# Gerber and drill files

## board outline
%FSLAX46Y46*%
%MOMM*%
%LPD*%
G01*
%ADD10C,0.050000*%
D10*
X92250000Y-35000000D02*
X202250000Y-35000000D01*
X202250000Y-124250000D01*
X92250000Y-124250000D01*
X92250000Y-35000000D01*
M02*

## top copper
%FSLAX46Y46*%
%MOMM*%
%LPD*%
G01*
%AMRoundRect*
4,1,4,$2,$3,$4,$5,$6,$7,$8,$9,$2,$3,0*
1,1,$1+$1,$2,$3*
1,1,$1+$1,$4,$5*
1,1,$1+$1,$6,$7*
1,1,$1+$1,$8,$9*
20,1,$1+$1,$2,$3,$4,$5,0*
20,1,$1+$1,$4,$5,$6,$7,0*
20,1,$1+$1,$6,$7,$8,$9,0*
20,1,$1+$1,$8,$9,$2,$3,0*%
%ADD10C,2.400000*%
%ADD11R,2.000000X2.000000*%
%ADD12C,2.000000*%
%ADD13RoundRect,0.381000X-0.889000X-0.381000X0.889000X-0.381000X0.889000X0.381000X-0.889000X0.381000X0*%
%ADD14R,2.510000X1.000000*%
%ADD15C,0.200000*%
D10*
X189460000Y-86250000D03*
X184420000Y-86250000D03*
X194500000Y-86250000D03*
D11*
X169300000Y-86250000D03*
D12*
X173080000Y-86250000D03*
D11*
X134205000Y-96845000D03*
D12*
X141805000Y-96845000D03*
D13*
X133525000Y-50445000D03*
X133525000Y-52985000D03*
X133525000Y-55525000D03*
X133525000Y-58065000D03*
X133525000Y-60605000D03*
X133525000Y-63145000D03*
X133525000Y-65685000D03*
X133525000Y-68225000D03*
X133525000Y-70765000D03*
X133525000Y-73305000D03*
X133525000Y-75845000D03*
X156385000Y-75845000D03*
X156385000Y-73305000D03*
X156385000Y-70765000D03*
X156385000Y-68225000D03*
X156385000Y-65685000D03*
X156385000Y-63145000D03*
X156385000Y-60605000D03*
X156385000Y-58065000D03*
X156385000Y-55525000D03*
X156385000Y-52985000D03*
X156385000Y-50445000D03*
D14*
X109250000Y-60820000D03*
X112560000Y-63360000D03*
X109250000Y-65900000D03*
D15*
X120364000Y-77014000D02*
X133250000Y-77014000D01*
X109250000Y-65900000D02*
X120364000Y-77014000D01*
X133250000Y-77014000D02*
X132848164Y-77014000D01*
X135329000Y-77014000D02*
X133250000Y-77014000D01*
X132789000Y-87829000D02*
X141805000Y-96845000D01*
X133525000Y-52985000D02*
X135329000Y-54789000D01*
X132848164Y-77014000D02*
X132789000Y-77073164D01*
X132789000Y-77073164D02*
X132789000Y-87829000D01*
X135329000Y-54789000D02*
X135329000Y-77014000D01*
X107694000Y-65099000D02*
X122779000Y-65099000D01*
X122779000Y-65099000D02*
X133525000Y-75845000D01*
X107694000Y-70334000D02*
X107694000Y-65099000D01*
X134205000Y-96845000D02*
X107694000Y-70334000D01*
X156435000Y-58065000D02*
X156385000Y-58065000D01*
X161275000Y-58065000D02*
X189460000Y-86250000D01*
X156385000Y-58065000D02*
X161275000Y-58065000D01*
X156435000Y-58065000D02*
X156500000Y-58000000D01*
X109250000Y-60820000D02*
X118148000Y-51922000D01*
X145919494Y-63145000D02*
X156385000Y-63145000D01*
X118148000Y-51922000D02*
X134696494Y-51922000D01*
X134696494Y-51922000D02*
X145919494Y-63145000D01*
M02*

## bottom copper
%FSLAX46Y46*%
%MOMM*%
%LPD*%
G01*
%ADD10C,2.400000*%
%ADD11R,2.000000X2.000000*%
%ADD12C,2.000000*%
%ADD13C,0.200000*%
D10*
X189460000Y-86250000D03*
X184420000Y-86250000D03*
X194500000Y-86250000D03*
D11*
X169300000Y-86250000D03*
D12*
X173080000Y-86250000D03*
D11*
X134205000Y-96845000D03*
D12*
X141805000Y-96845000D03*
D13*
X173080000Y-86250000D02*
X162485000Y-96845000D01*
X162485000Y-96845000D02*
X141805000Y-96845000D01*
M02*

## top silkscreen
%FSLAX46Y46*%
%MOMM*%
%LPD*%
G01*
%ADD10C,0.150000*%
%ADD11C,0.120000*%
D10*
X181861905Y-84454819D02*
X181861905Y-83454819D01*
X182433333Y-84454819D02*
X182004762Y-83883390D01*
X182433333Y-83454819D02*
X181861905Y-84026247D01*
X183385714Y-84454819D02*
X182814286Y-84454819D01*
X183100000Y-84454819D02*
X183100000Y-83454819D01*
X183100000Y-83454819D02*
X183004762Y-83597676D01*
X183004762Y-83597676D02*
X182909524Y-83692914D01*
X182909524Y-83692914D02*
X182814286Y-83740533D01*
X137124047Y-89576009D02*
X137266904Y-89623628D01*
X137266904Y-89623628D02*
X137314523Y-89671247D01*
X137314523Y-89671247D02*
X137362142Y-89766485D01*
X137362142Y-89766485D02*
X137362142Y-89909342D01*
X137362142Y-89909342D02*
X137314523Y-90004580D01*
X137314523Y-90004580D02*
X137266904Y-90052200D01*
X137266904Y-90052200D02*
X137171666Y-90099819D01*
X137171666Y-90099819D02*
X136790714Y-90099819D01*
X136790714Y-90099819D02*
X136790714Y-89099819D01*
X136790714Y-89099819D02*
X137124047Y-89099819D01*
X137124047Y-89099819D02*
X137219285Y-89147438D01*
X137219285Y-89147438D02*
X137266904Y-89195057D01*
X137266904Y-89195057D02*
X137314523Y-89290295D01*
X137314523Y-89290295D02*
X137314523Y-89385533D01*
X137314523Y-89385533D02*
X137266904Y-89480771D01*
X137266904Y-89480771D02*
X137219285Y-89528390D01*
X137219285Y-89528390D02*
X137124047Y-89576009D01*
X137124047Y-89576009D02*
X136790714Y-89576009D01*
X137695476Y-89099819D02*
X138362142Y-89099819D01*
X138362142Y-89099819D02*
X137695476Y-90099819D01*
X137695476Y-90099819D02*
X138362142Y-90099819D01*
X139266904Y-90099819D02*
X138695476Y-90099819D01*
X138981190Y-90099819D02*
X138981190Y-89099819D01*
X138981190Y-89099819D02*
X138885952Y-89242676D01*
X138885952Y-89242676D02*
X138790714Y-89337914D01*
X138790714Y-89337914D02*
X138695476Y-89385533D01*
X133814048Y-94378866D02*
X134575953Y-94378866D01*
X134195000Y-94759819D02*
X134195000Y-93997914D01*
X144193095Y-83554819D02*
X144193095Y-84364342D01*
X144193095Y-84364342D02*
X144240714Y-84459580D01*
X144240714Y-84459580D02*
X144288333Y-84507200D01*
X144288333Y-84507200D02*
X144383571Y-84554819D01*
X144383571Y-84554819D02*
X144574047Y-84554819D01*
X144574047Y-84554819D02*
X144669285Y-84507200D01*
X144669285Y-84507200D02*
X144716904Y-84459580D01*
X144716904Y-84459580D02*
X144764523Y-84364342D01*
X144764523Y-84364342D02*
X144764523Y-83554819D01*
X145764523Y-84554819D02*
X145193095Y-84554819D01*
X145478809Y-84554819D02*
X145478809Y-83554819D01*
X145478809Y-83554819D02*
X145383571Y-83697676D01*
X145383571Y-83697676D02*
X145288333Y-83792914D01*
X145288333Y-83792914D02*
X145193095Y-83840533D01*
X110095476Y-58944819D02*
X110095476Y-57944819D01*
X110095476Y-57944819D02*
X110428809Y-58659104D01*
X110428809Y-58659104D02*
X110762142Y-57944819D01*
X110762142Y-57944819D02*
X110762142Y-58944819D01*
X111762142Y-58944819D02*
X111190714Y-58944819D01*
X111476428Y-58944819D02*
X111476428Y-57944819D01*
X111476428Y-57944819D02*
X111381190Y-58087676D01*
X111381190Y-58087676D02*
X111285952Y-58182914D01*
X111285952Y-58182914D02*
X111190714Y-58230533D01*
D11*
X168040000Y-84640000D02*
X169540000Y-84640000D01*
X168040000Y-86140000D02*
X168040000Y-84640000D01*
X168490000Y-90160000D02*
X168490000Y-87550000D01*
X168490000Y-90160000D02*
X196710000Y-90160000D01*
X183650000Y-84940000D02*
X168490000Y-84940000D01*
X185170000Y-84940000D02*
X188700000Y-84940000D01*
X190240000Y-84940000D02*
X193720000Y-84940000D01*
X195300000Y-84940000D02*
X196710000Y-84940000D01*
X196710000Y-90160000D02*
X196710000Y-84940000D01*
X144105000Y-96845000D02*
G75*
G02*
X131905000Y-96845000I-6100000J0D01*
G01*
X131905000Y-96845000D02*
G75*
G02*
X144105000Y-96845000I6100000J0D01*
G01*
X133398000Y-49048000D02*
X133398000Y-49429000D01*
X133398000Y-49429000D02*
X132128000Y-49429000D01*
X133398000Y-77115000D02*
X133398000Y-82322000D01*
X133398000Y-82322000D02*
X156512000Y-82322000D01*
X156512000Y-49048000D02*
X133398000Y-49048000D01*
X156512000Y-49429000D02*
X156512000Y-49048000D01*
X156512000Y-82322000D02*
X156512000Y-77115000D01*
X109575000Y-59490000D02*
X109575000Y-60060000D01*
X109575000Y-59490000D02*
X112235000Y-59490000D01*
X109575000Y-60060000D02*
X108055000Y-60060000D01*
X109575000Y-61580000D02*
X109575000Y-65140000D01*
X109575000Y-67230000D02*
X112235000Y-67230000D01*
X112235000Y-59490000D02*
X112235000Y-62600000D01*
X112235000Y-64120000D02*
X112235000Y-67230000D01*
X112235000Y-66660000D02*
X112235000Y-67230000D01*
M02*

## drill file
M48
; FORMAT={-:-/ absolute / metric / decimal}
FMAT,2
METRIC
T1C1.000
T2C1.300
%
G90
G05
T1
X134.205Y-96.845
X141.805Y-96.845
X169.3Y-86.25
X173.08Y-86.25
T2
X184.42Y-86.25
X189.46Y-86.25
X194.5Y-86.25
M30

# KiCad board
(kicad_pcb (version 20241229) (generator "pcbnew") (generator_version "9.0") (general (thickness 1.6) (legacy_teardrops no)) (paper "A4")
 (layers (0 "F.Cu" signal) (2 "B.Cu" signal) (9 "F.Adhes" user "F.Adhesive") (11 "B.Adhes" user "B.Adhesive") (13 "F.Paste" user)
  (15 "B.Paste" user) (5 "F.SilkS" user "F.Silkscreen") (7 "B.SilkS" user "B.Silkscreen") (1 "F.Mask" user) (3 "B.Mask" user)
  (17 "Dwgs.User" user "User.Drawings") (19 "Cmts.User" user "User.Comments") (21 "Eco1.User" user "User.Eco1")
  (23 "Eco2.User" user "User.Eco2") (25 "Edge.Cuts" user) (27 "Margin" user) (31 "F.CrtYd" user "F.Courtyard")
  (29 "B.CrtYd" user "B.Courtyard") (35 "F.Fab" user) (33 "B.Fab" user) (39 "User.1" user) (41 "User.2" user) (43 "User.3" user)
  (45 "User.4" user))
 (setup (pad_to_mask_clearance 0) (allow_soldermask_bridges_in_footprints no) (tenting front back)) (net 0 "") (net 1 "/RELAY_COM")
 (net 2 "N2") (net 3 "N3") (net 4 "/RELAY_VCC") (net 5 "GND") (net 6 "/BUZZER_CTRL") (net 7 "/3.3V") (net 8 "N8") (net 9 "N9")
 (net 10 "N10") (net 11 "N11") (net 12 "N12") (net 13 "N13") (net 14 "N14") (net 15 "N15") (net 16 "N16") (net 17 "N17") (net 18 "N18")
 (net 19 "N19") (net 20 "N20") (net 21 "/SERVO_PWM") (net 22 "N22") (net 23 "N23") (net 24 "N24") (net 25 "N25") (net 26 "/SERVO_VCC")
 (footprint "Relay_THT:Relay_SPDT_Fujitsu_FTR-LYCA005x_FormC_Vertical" (layer "F.Cu") (at 169.3 86.25)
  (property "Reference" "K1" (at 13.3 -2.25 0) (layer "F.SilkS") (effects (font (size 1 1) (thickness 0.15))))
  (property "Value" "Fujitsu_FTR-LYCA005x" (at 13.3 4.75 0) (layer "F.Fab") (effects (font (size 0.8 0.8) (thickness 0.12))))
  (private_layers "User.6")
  (fp_line (start -1.26 -1.61) (end 0.24 -1.61) (stroke (width 0.12) (type solid)) (layer "F.SilkS"))
  (fp_line (start -1.26 -0.11) (end -1.26 -1.61) (stroke (width 0.12) (type solid)) (layer "F.SilkS"))
  (fp_line (start -0.81 3.91) (end -0.81 1.3) (stroke (width 0.12) (type solid)) (layer "F.SilkS"))
  (fp_line (start -0.81 3.91) (end 27.41 3.91) (stroke (width 0.12) (type solid)) (layer "F.SilkS"))
  (fp_line (start 14.35 -1.31) (end -0.81 -1.31) (stroke (width 0.12) (type solid)) (layer "F.SilkS"))
  (fp_line (start 15.87 -1.31) (end 19.4 -1.31) (stroke (width 0.12) (type solid)) (layer "F.SilkS"))
  (fp_line (start 20.94 -1.31) (end 24.42 -1.31) (stroke (width 0.12) (type solid)) (layer "F.SilkS"))
  (fp_line (start 26 -1.31) (end 27.41 -1.31) (stroke (width 0.12) (type solid)) (layer "F.SilkS"))
  (fp_line (start 27.41 3.91) (end 27.41 -1.31) (stroke (width 0.12) (type solid)) (layer "F.SilkS"))
  (pad "11" thru_hole circle (at 20.16 0) (size 2.4 2.4) (drill 1.3) (layers "*.Cu" "*.Mask") (remove_unused_layers no) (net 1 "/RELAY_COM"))
  (pad "12" thru_hole circle (at 15.12 0) (size 2.4 2.4) (drill 1.3) (layers "*.Cu" "*.Mask") (remove_unused_layers no) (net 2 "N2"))
  (pad "14" thru_hole circle (at 25.2 0) (size 2.4 2.4) (drill 1.3) (layers "*.Cu" "*.Mask") (remove_unused_layers no) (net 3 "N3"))
  (pad "A1" thru_hole rect (at 0 0) (size 2 2) (drill 1) (layers "*.Cu" "*.Mask") (remove_unused_layers no) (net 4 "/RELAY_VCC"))
  (pad "A2" thru_hole circle (at 3.78 0) (size 2 2) (drill 1) (layers "*.Cu" "*.Mask") (remove_unused_layers no) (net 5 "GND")))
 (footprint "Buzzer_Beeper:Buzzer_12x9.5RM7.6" (layer "F.Cu") (at 134.205 96.845)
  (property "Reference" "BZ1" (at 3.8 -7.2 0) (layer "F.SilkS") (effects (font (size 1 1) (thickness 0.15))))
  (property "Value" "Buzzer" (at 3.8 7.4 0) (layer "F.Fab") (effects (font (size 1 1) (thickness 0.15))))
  (fp_circle (center 3.8 0) (end 9.9 0) (stroke (width 0.12) (type solid)) (fill no) (layer "F.SilkS"))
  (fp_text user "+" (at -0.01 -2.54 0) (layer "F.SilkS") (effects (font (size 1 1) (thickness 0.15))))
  (pad "1" thru_hole rect (at 0 0) (size 2 2) (drill 1) (layers "*.Cu" "*.Mask") (remove_unused_layers no) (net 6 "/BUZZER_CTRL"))
  (pad "2" thru_hole circle (at 7.6 0) (size 2 2) (drill 1) (layers "*.Cu" "*.Mask") (remove_unused_layers no) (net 5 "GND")))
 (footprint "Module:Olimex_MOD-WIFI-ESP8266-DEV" (layer "F.Cu") (at 144.955 63.145)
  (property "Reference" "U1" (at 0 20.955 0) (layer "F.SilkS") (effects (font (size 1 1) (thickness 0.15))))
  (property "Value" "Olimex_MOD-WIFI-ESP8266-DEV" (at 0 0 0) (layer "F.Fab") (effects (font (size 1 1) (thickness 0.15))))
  (fp_line (start -11.557 -14.097) (end -11.557 -13.716) (stroke (width 0.12) (type solid)) (layer "F.SilkS"))
  (fp_line (start -11.557 -13.716) (end -12.827 -13.716) (stroke (width 0.12) (type solid)) (layer "F.SilkS"))
  (fp_line (start -11.557 13.97) (end -11.557 19.177) (stroke (width 0.12) (type solid)) (layer "F.SilkS"))
  (fp_line (start -11.557 19.177) (end 11.557 19.177) (stroke (width 0.12) (type solid)) (layer "F.SilkS"))
  (fp_line (start 11.557 -14.097) (end -11.557 -14.097) (stroke (width 0.12) (type solid)) (layer "F.SilkS"))
  (fp_line (start 11.557 -13.716) (end 11.557 -14.097) (stroke (width 0.12) (type solid)) (layer "F.SilkS"))
  (fp_line (start 11.557 19.177) (end 11.557 13.97) (stroke (width 0.12) (type solid)) (layer "F.SilkS"))
  (pad "1" smd roundrect (at -11.43 -12.7) (size 2.54 1.524) (layers "F.Cu" "F.Mask" "F.Paste") (roundrect_rratio 0.25) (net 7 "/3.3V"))
  (pad "2" smd roundrect (at -11.43 -10.16) (size 2.54 1.524) (layers "F.Cu" "F.Mask" "F.Paste") (roundrect_rratio 0.25) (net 5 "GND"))
  (pad "3" smd roundrect (at -11.43 -7.62) (size 2.54 1.524) (layers "F.Cu" "F.Mask" "F.Paste") (roundrect_rratio 0.25) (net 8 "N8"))
  (pad "4" smd roundrect (at -11.43 -5.08) (size 2.54 1.524) (layers "F.Cu" "F.Mask" "F.Paste") (roundrect_rratio 0.25) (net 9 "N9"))
  (pad "5" smd roundrect (at -11.43 -2.54) (size 2.54 1.524) (layers "F.Cu" "F.Mask" "F.Paste") (roundrect_rratio 0.25) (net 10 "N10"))
  (pad "6" smd roundrect (at -11.43 0) (size 2.54 1.524) (layers "F.Cu" "F.Mask" "F.Paste") (roundrect_rratio 0.25) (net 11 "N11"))
  (pad "7" smd roundrect (at -11.43 2.54) (size 2.54 1.524) (layers "F.Cu" "F.Mask" "F.Paste") (roundrect_rratio 0.25) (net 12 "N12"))
  (pad "8" smd roundrect (at -11.43 5.08) (size 2.54 1.524) (layers "F.Cu" "F.Mask" "F.Paste") (roundrect_rratio 0.25) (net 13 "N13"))
  (pad "9" smd roundrect (at -11.43 7.62) (size 2.54 1.524) (layers "F.Cu" "F.Mask" "F.Paste") (roundrect_rratio 0.25) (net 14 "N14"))
  (pad "10" smd roundrect (at -11.43 10.16) (size 2.54 1.524) (layers "F.Cu" "F.Mask" "F.Paste") (roundrect_rratio 0.25) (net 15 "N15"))
  (pad "11" smd roundrect (at -11.43 12.7) (size 2.54 1.524) (layers "F.Cu" "F.Mask" "F.Paste") (roundrect_rratio 0.25)
   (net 6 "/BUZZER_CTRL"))
  (pad "12" smd roundrect (at 11.43 12.7) (size 2.54 1.524) (layers "F.Cu" "F.Mask" "F.Paste") (roundrect_rratio 0.25) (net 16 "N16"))
  (pad "13" smd roundrect (at 11.43 10.16) (size 2.54 1.524) (layers "F.Cu" "F.Mask" "F.Paste") (roundrect_rratio 0.25) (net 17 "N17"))
  (pad "14" smd roundrect (at 11.43 7.62) (size 2.54 1.524) (layers "F.Cu" "F.Mask" "F.Paste") (roundrect_rratio 0.25) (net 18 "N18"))
  (pad "15" smd roundrect (at 11.43 5.08) (size 2.54 1.524) (layers "F.Cu" "F.Mask" "F.Paste") (roundrect_rratio 0.25) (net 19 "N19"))
  (pad "16" smd roundrect (at 11.43 2.54) (size 2.54 1.524) (layers "F.Cu" "F.Mask" "F.Paste") (roundrect_rratio 0.25) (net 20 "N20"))
  (pad "17" smd roundrect (at 11.43 0) (size 2.54 1.524) (layers "F.Cu" "F.Mask" "F.Paste") (roundrect_rratio 0.25) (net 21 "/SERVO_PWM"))
  (pad "18" smd roundrect (at 11.43 -2.54) (size 2.54 1.524) (layers "F.Cu" "F.Mask" "F.Paste") (roundrect_rratio 0.25) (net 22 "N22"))
  (pad "19" smd roundrect (at 11.43 -5.08) (size 2.54 1.524) (layers "F.Cu" "F.Mask" "F.Paste") (roundrect_rratio 0.25) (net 1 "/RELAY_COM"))
  (pad "20" smd roundrect (at 11.43 -7.62) (size 2.54 1.524) (layers "F.Cu" "F.Mask" "F.Paste") (roundrect_rratio 0.25) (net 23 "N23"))
  (pad "21" smd roundrect (at 11.43 -10.16) (size 2.54 1.524) (layers "F.Cu" "F.Mask" "F.Paste") (roundrect_rratio 0.25) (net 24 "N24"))
  (pad "22" smd roundrect (at 11.43 -12.7) (size 2.54 1.524) (layers "F.Cu" "F.Mask" "F.Paste") (roundrect_rratio 0.25) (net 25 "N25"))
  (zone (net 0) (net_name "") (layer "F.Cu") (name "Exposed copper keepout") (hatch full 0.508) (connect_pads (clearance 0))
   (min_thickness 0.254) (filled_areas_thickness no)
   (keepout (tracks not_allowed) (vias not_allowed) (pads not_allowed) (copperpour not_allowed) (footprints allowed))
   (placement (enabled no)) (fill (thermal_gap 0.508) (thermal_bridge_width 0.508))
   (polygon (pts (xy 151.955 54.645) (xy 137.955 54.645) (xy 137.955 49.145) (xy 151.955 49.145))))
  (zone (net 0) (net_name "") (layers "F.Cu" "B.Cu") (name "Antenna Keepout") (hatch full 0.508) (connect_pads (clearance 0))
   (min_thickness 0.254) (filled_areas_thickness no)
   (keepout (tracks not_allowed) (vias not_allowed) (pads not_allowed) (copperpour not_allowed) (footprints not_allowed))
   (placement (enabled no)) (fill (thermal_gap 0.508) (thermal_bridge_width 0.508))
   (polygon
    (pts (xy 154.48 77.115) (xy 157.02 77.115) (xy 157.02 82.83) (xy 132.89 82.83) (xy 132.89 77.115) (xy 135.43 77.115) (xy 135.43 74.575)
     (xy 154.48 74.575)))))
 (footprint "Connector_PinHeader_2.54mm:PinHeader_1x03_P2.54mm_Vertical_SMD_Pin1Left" (layer "F.Cu") (at 110.905 63.36)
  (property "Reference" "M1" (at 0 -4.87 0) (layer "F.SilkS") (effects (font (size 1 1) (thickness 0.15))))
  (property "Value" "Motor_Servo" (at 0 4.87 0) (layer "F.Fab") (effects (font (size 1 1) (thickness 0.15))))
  (fp_line (start -1.33 -3.87) (end -1.33 -3.3) (stroke (width 0.12) (type solid)) (layer "F.SilkS"))
  (fp_line (start -1.33 -3.87) (end 1.33 -3.87) (stroke (width 0.12) (type solid)) (layer "F.SilkS"))
  (fp_line (start -1.33 -3.3) (end -2.85 -3.3) (stroke (width 0.12) (type solid)) (layer "F.SilkS"))
  (fp_line (start -1.33 -1.78) (end -1.33 1.78) (stroke (width 0.12) (type solid)) (layer "F.SilkS"))
  (fp_line (start -1.33 3.87) (end 1.33 3.87) (stroke (width 0.12) (type solid)) (layer "F.SilkS"))
  (fp_line (start 1.33 -3.87) (end 1.33 -0.76) (stroke (width 0.12) (type solid)) (layer "F.SilkS"))
  (fp_line (start 1.33 0.76) (end 1.33 3.87) (stroke (width 0.12) (type solid)) (layer "F.SilkS"))
  (fp_line (start 1.33 3.3) (end 1.33 3.87) (stroke (width 0.12) (type solid)) (layer "F.SilkS"))
  (pad "1" smd rect (at -1.655 -2.54) (size 2.51 1) (layers "F.Cu" "F.Mask" "F.Paste") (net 21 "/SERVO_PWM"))
  (pad "2" smd rect (at 1.655 0) (size 2.51 1) (layers "F.Cu" "F.Mask" "F.Paste") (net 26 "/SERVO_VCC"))
  (pad "3" smd rect (at -1.655 2.54) (size 2.51 1) (layers "F.Cu" "F.Mask" "F.Paste") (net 5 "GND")))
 (gr_rect (start 92.25 35) (end 202.25 124.25) (stroke (width 0.05) (type default)) (fill no) (layer "Edge.Cuts"))
 (segment (start 120.364 77.014) (end 133.25 77.014) (width 0.2) (layer "F.Cu") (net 5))
 (segment (start 109.25 65.9) (end 120.364 77.014) (width 0.2) (layer "F.Cu") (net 5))
 (segment (start 133.25 77.014) (end 132.848164 77.014) (width 0.2) (layer "F.Cu") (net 5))
 (segment (start 135.329 77.014) (end 133.25 77.014) (width 0.2) (layer "F.Cu") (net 5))
 (segment (start 132.789 87.829) (end 141.805 96.845) (width 0.2) (layer "F.Cu") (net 5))
 (segment (start 133.525 52.985) (end 135.329 54.789) (width 0.2) (layer "F.Cu") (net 5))
 (segment (start 132.848164 77.014) (end 132.789 77.073164) (width 0.2) (layer "F.Cu") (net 5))
 (segment (start 132.789 77.073164) (end 132.789 87.829) (width 0.2) (layer "F.Cu") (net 5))
 (segment (start 135.329 54.789) (end 135.329 77.014) (width 0.2) (layer "F.Cu") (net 5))
 (segment (start 173.08 86.25) (end 162.485 96.845) (width 0.2) (layer "B.Cu") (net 5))
 (segment (start 162.485 96.845) (end 141.805 96.845) (width 0.2) (layer "B.Cu") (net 5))
 (segment (start 107.694 65.099) (end 122.779 65.099) (width 0.2) (layer "F.Cu") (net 6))
 (segment (start 122.779 65.099) (end 133.525 75.845) (width 0.2) (layer "F.Cu") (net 6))
 (segment (start 107.694 70.334) (end 107.694 65.099) (width 0.2) (layer "F.Cu") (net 6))
 (segment (start 134.205 96.845) (end 107.694 70.334) (width 0.2) (layer "F.Cu") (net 6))
 (segment (start 156.435 58.065) (end 156.385 58.065) (width 0.2) (layer "F.Cu") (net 1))
 (segment (start 161.275 58.065) (end 189.46 86.25) (width 0.2) (layer "F.Cu") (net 1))
 (segment (start 156.385 58.065) (end 161.275 58.065) (width 0.2) (layer "F.Cu") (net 1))
 (segment (start 156.435 58.065) (end 156.5 58) (width 0.2) (layer "F.Cu") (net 1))
 (segment (start 109.25 60.82) (end 118.148 51.922) (width 0.2) (layer "F.Cu") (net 21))
 (segment (start 145.919494 63.145) (end 156.385 63.145) (width 0.2) (layer "F.Cu") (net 21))
 (segment (start 118.148 51.922) (end 134.696494 51.922) (width 0.2) (layer "F.Cu") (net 21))
 (segment (start 134.696494 51.922) (end 145.919494 63.145) (width 0.2) (layer "F.Cu") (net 21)))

